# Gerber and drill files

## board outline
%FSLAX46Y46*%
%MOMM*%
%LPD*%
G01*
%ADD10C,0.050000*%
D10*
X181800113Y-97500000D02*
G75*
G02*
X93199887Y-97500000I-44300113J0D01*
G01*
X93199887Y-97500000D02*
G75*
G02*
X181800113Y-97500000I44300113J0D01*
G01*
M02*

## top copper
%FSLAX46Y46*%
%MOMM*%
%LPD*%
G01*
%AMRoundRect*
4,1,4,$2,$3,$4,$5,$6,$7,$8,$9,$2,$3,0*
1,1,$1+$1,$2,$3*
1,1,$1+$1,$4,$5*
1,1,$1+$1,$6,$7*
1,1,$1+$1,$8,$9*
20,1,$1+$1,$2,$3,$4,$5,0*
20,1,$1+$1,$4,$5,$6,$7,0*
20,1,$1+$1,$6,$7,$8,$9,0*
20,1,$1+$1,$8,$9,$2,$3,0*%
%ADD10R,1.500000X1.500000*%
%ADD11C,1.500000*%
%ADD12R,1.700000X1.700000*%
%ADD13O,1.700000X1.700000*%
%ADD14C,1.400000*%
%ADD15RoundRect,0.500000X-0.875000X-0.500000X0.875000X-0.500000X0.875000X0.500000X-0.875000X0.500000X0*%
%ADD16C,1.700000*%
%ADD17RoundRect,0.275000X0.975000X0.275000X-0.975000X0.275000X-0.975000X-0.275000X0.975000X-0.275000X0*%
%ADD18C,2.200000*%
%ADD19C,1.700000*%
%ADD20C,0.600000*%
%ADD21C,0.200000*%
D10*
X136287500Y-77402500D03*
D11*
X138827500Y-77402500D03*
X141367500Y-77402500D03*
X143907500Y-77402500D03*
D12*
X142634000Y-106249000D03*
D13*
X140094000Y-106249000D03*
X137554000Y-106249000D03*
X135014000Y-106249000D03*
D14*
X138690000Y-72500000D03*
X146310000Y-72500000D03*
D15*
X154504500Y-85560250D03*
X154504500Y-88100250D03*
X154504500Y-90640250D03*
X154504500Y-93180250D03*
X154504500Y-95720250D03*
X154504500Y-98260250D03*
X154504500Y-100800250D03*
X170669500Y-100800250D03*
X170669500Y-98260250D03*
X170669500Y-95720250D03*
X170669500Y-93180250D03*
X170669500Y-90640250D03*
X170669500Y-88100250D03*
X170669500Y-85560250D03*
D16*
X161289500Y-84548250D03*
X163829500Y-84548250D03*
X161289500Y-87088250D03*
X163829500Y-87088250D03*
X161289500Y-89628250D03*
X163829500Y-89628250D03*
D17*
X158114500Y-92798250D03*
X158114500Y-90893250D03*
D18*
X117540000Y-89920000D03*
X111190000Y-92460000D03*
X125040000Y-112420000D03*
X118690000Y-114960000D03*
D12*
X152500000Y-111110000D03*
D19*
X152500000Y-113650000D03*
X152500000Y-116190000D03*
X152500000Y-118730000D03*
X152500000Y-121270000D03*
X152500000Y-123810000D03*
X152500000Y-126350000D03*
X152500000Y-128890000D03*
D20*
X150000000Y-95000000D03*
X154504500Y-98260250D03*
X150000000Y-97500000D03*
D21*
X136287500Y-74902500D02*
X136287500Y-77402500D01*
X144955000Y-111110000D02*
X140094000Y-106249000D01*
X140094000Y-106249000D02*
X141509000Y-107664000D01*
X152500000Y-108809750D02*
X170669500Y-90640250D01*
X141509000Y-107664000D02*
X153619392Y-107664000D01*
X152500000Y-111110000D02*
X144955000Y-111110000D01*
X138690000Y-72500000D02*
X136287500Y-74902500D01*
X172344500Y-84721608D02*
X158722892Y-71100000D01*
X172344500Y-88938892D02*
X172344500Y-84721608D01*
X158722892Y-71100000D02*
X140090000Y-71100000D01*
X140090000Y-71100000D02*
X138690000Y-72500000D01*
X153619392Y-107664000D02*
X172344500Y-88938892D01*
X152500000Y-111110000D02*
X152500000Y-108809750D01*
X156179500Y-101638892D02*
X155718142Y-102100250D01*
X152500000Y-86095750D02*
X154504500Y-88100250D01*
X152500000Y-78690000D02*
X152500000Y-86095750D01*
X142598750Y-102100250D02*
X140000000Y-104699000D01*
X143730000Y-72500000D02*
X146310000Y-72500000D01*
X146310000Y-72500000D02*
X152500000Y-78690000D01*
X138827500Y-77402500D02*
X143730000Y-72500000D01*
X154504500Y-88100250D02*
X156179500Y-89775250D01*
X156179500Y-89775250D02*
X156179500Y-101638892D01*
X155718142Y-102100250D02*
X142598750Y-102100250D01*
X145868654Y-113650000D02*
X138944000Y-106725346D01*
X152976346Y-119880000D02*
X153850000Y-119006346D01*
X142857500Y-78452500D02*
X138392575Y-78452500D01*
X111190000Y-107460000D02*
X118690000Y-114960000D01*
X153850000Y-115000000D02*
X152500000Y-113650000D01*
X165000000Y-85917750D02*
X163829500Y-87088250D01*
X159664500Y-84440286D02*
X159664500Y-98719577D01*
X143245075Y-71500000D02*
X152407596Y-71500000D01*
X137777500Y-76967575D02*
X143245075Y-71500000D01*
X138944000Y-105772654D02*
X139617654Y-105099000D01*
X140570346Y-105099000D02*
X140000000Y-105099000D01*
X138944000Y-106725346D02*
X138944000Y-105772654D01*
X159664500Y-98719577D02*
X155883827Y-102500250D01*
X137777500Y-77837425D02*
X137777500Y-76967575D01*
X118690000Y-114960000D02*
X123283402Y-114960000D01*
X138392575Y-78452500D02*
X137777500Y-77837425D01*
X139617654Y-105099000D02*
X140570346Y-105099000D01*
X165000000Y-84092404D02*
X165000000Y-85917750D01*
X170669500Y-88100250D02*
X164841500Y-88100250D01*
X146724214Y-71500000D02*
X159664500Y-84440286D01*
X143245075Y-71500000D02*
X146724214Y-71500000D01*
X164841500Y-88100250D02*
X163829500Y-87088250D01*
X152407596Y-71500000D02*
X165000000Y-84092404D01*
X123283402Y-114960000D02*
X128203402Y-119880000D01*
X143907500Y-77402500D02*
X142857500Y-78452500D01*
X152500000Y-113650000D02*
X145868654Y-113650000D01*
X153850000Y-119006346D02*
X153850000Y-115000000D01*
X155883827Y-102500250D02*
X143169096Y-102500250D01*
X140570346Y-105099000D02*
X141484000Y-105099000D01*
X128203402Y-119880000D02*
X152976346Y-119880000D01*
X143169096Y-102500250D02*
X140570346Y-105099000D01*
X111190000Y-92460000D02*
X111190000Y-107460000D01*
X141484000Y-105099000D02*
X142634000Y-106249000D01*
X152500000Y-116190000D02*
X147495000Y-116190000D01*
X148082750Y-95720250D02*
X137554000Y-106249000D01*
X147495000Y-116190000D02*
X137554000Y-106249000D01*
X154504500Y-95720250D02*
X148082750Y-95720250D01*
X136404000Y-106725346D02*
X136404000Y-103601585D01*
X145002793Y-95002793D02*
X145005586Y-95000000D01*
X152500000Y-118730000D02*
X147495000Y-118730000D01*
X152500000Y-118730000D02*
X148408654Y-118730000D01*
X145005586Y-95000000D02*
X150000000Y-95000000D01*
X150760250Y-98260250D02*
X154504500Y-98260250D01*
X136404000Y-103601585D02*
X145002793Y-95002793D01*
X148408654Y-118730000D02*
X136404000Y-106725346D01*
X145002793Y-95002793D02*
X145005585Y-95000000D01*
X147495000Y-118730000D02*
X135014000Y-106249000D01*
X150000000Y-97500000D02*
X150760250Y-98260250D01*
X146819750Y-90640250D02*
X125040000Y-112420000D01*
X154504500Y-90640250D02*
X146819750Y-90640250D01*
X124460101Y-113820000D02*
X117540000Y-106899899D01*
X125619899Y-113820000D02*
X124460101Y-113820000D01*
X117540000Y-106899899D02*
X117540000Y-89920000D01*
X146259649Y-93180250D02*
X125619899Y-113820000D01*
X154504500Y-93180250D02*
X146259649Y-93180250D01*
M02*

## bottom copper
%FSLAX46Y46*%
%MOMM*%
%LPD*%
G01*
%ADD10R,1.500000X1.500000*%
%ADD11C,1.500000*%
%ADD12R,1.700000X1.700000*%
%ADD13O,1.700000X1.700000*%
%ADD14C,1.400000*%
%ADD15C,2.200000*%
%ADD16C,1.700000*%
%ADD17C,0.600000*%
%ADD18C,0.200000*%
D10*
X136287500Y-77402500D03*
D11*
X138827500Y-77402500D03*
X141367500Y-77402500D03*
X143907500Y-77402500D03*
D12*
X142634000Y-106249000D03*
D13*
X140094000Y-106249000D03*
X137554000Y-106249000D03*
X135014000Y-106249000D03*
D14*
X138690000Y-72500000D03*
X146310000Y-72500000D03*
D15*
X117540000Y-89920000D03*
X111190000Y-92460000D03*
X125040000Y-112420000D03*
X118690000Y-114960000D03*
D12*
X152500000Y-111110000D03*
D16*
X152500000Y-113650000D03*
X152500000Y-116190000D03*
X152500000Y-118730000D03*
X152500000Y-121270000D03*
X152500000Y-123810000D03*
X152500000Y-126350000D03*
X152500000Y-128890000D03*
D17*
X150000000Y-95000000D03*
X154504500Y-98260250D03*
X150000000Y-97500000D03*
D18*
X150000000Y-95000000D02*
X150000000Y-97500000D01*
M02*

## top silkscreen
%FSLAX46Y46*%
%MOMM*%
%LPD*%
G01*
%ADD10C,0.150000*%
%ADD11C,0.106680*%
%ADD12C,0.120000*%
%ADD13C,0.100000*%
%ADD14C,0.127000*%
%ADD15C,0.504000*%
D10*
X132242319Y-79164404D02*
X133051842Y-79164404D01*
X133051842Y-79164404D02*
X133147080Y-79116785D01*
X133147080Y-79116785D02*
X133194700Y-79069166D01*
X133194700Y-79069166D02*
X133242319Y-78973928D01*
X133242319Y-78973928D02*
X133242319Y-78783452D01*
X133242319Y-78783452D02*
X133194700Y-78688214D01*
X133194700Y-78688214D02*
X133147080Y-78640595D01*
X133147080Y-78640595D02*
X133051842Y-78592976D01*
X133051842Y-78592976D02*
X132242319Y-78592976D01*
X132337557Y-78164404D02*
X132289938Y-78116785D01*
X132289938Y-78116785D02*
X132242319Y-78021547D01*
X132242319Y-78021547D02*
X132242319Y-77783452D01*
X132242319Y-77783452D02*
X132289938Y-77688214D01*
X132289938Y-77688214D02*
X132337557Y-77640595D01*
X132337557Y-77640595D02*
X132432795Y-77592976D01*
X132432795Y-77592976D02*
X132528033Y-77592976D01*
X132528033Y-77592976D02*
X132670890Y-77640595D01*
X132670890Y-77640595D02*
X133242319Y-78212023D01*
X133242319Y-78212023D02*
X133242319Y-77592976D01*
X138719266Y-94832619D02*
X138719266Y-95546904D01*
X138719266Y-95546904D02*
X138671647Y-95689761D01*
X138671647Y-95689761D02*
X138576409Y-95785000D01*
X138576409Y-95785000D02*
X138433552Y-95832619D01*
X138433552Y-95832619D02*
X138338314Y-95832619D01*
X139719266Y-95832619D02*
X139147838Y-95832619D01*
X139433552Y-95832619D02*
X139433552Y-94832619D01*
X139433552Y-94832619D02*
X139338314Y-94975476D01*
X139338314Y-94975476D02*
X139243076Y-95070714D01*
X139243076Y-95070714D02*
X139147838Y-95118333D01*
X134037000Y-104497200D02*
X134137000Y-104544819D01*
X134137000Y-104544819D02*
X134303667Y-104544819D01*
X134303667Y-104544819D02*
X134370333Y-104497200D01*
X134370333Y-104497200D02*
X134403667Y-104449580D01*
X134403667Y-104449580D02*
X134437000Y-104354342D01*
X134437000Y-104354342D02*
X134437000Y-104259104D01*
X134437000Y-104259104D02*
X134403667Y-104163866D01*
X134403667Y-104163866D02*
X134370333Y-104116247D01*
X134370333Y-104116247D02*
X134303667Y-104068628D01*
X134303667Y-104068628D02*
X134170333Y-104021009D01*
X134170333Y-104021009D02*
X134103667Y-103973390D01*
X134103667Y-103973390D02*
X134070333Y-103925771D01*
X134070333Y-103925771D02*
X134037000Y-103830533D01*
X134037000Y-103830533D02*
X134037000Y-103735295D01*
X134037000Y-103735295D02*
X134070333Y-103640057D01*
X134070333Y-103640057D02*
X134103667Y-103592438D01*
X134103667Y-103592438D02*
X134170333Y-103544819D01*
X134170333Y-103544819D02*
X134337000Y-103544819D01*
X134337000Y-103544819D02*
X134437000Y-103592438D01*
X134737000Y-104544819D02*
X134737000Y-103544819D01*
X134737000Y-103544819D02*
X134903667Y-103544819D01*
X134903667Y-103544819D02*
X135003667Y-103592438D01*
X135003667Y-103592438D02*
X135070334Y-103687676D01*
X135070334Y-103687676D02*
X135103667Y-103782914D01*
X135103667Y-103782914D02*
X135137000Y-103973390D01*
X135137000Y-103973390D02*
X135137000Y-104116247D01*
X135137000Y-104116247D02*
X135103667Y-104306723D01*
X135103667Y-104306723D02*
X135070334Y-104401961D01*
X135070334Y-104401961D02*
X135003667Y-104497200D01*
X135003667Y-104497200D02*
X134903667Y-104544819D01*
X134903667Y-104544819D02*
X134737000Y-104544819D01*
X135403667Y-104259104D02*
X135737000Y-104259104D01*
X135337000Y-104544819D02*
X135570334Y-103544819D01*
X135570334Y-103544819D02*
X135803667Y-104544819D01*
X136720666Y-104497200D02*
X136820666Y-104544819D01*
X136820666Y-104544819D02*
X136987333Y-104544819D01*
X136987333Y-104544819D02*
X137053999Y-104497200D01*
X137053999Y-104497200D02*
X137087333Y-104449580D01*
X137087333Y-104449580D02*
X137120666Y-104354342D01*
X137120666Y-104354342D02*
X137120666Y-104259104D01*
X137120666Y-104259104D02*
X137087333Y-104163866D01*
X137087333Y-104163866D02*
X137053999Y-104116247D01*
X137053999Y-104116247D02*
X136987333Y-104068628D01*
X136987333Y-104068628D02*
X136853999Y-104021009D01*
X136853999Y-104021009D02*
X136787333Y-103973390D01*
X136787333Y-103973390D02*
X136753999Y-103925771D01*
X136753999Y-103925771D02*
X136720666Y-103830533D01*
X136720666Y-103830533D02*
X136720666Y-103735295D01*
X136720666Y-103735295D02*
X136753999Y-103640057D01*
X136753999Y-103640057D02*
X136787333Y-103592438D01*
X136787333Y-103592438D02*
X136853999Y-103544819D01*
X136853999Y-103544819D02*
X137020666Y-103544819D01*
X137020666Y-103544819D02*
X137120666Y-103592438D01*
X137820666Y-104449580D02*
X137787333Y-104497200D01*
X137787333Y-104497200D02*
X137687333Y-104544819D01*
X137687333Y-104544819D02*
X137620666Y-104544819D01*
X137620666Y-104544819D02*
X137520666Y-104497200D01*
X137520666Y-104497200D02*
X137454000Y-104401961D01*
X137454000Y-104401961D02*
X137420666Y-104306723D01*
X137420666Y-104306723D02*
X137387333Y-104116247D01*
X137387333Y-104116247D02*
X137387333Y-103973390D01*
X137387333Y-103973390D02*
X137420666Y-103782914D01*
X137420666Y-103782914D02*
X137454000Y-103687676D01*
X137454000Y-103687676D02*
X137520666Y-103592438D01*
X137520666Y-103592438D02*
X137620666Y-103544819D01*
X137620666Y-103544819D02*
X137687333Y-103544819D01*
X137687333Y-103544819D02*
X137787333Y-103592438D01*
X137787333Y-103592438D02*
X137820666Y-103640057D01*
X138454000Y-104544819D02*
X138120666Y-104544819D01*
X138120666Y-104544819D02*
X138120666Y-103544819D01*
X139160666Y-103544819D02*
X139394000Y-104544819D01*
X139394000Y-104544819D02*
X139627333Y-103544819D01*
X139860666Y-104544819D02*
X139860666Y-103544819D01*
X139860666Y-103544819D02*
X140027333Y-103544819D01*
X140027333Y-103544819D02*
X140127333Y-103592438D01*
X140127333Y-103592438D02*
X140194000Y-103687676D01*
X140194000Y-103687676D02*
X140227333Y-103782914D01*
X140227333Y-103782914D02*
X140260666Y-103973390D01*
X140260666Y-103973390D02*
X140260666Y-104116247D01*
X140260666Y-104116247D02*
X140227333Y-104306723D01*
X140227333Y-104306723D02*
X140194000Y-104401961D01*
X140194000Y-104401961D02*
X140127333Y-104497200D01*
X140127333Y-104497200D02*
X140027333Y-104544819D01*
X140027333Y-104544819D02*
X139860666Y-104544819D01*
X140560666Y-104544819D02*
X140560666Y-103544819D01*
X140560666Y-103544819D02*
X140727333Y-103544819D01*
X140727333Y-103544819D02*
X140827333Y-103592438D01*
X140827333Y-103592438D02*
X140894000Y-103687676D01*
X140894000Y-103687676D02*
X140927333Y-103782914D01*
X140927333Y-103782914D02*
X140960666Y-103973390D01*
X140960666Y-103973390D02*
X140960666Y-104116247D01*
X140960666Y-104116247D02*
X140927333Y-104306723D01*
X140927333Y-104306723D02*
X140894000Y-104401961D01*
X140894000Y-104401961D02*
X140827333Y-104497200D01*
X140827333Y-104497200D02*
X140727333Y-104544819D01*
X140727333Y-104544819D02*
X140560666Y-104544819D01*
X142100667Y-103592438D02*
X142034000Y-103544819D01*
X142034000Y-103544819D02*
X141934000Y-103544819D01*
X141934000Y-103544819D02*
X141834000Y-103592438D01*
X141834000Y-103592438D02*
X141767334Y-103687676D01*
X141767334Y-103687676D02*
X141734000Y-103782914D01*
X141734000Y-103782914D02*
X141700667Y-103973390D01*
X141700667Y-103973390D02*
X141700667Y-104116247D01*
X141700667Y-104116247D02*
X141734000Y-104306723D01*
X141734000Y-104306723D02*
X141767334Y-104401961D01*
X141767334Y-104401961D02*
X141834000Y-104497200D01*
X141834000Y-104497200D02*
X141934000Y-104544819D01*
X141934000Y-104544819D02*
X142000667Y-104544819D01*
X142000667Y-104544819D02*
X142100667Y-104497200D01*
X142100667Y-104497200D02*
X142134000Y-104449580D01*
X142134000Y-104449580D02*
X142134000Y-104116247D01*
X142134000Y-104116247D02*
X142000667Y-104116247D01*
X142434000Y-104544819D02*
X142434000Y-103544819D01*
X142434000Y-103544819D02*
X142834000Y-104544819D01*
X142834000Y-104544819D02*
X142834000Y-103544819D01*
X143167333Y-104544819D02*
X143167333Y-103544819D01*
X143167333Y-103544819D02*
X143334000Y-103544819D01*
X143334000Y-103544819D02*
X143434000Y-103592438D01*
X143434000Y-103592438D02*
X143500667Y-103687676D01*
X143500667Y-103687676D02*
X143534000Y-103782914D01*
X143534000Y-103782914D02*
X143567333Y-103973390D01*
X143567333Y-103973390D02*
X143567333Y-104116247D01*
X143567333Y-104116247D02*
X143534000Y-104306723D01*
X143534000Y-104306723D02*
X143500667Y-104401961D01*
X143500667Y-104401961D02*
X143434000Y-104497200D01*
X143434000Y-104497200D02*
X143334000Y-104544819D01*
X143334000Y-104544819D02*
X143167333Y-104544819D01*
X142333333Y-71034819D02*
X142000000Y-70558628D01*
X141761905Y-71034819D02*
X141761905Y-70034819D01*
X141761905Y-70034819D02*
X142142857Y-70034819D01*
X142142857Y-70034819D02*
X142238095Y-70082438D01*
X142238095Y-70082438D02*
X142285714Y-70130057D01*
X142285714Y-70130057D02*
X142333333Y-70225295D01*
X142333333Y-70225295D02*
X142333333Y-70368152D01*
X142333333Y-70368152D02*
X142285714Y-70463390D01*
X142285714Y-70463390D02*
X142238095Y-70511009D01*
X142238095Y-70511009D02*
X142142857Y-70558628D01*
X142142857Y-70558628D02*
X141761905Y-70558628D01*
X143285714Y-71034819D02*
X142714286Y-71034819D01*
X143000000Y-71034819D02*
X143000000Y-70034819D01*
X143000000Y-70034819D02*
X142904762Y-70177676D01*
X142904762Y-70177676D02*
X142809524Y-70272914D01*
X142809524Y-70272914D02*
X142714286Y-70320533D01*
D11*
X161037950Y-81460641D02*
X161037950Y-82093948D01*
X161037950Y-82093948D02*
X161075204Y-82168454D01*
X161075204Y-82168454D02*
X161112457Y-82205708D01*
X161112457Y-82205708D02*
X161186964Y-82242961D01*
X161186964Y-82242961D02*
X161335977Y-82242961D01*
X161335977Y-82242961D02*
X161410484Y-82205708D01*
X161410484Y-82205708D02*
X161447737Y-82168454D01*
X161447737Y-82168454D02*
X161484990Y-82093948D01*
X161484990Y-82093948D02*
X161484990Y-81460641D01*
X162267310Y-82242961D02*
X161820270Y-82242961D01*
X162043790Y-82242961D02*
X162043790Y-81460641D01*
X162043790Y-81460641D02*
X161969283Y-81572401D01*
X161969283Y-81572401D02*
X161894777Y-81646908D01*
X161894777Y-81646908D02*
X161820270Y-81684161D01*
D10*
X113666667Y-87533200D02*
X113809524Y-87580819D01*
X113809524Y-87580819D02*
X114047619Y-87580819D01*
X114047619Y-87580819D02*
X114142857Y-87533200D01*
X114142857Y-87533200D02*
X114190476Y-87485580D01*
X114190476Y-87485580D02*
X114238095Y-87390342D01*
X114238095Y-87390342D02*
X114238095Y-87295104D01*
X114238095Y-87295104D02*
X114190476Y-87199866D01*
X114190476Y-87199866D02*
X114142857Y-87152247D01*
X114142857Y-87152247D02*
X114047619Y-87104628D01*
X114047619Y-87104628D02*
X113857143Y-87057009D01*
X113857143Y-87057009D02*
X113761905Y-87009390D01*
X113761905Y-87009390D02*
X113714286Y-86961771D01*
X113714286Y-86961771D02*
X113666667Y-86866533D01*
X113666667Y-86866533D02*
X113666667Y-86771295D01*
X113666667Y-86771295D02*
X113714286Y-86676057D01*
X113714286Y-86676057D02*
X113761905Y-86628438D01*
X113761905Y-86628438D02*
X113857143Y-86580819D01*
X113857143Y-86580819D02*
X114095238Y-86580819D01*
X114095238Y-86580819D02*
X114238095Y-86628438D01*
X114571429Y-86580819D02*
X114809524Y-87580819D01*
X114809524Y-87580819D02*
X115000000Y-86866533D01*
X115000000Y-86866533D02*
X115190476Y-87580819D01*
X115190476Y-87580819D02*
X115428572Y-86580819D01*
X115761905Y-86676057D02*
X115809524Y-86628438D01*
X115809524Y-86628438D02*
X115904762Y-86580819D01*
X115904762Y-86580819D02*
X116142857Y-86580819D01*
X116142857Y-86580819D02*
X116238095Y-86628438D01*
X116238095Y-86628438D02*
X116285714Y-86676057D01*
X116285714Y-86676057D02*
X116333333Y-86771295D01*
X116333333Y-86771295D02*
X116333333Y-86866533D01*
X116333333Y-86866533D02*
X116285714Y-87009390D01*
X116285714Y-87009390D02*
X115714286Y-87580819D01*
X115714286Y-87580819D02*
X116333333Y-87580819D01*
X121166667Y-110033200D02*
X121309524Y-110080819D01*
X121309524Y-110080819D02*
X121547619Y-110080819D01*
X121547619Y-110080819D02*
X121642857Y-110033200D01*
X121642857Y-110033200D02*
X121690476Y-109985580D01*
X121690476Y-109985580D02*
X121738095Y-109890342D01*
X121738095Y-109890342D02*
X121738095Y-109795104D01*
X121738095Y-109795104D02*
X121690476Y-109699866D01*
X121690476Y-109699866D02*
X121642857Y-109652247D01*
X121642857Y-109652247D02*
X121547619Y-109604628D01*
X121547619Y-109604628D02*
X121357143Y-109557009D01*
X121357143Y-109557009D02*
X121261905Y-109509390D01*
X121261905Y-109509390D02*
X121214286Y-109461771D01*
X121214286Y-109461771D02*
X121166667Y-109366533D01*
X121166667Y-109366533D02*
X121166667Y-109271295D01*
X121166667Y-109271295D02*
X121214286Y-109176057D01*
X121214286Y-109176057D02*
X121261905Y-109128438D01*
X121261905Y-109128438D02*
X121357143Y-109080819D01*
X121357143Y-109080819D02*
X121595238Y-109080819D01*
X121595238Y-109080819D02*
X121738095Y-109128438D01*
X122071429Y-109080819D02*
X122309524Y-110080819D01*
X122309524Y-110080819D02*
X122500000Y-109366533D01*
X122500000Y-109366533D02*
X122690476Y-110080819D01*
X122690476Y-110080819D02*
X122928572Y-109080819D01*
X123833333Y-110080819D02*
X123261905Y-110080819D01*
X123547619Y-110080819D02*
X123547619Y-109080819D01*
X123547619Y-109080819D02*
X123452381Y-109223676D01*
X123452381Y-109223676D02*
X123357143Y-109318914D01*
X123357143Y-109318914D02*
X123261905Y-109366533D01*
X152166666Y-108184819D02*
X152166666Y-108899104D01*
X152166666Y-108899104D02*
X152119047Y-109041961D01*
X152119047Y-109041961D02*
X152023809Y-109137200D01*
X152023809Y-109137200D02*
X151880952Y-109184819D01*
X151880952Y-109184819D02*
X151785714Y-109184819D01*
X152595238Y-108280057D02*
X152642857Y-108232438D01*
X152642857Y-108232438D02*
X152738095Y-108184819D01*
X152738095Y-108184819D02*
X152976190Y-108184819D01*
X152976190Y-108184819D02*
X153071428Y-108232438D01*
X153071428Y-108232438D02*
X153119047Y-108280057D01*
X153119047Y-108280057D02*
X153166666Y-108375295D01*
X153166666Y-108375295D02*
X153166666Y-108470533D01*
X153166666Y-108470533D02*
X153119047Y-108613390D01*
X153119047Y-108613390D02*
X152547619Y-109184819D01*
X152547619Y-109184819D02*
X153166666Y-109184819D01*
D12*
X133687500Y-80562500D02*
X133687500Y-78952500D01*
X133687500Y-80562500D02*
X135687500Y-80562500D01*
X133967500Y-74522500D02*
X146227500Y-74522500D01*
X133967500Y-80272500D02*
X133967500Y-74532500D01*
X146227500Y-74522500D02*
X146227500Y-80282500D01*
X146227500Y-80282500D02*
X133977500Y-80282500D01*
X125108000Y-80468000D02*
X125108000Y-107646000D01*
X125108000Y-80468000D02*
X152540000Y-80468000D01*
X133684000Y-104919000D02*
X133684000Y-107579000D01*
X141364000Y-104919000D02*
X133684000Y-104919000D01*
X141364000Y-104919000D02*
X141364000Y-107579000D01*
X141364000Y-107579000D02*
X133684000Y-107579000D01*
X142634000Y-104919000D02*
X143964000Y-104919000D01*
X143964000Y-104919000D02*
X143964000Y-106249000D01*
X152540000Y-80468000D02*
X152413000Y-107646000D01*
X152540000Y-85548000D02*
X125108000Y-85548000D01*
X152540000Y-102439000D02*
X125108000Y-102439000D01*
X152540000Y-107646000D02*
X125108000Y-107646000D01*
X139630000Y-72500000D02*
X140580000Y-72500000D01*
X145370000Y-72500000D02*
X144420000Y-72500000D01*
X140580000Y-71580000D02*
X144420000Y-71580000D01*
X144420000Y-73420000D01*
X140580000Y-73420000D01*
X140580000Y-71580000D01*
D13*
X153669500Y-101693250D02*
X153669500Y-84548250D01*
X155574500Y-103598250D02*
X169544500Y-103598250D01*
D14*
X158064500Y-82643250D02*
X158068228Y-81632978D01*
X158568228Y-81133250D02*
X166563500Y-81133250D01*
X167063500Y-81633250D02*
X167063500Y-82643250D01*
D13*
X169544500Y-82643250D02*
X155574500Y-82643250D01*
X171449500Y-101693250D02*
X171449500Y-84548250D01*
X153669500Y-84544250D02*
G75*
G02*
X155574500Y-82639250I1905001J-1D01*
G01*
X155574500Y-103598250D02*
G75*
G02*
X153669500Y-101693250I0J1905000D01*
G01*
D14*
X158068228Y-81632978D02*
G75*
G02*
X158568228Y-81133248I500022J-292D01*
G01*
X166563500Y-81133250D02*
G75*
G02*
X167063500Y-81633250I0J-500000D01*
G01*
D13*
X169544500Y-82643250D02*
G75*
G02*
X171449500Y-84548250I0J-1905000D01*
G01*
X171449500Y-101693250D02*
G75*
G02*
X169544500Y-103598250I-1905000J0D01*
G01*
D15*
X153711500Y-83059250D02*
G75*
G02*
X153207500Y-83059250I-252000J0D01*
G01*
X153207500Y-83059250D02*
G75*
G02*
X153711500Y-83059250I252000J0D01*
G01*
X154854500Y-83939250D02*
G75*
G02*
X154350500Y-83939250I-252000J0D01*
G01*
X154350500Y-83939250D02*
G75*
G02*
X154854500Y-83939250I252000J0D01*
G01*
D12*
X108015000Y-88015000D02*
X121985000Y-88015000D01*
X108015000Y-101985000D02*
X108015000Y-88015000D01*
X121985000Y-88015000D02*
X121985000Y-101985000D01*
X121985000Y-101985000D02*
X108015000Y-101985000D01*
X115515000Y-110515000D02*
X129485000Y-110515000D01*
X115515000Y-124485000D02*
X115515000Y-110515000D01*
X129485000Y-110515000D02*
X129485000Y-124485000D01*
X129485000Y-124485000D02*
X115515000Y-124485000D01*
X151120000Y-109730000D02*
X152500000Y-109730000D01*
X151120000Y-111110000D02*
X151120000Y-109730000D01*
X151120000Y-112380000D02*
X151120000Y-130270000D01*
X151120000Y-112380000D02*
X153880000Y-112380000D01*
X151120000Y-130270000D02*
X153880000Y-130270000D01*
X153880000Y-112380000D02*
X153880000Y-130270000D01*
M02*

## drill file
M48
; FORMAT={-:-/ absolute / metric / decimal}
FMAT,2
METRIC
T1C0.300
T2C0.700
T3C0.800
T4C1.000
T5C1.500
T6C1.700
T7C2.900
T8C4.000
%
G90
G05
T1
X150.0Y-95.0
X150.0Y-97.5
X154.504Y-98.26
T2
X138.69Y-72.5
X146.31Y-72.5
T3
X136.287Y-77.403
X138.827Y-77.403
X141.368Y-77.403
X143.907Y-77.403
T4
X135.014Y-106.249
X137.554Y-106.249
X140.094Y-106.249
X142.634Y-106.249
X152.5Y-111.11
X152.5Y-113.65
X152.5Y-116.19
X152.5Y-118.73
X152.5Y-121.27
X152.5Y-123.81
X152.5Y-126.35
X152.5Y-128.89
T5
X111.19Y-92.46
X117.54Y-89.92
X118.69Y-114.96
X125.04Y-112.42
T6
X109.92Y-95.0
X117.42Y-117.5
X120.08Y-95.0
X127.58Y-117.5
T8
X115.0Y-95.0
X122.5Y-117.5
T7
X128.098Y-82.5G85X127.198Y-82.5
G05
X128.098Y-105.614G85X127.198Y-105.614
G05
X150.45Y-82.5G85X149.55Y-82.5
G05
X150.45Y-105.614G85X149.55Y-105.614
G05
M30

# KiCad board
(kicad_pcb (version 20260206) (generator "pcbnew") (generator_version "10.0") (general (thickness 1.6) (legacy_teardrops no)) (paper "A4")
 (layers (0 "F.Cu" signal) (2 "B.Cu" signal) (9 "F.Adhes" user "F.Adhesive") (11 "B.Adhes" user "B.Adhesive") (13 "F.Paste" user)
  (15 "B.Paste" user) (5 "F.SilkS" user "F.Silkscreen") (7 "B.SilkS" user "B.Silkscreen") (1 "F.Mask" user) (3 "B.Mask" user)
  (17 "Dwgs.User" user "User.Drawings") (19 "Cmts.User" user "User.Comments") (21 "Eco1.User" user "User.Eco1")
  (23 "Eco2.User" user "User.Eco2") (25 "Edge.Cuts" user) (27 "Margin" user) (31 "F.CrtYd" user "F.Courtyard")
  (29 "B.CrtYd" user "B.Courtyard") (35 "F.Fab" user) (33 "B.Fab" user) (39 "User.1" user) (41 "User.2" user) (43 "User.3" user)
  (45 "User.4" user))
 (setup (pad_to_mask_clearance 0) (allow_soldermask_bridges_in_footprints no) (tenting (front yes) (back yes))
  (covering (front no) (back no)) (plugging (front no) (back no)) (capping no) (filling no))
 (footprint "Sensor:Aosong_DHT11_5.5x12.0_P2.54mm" (layer "F.Cu") (at 136.2875 77.4025 90)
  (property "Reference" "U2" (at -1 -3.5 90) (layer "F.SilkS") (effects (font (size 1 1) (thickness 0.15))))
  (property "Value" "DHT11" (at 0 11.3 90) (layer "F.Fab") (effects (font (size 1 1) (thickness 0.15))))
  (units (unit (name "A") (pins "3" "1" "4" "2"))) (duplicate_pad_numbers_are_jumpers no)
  (fp_line (start -3.16 -2.6) (end -1.55 -2.6) (stroke (width 0.12) (type solid)) (layer "F.SilkS"))
  (fp_line (start -3.16 -2.6) (end -3.16 -0.6) (stroke (width 0.12) (type solid)) (layer "F.SilkS"))
  (fp_line (start 2.88 -2.32) (end 2.88 9.94) (stroke (width 0.12) (type solid)) (layer "F.SilkS"))
  (fp_line (start -2.87 -2.32) (end 2.87 -2.32) (stroke (width 0.12) (type solid)) (layer "F.SilkS"))
  (fp_line (start 2.88 9.94) (end -2.88 9.94) (stroke (width 0.12) (type solid)) (layer "F.SilkS"))
  (fp_line (start -2.88 9.94) (end -2.88 -2.31) (stroke (width 0.12) (type solid)) (layer "F.SilkS"))
  (pad "1" thru_hole rect (at 0 0 90) (size 1.5 1.5) (drill 0.8) (layers "*.Cu" "*.Mask") (remove_unused_layers no) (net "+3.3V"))
  (pad "2" thru_hole circle (at 0 2.54 90) (size 1.5 1.5) (drill 0.8) (layers "*.Cu" "*.Mask") (remove_unused_layers no) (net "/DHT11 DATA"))
  (pad "3" thru_hole circle (at 0 5.08 90) (size 1.5 1.5) (drill 0.8) (layers "*.Cu" "*.Mask") (remove_unused_layers no)
   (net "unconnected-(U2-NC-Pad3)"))
  (pad "4" thru_hole circle (at 0 7.62 90) (size 1.5 1.5) (drill 0.8) (layers "*.Cu" "*.Mask") (remove_unused_layers no) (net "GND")))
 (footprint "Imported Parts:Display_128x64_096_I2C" (layer "F.Cu") (at 138.824 106.249 180)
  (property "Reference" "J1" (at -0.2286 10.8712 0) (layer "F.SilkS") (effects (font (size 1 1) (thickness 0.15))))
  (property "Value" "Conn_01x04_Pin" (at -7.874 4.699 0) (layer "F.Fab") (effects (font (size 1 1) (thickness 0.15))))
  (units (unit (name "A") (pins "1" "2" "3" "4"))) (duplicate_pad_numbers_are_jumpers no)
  (fp_line (start 13.716 25.781) (end 13.716 -1.397) (stroke (width 0.12) (type solid)) (layer "F.SilkS"))
  (fp_line (start 13.716 25.781) (end -13.716 25.781) (stroke (width 0.12) (type solid)) (layer "F.SilkS"))
  (fp_line (start 5.14 1.33) (end 5.14 -1.33) (stroke (width 0.12) (type solid)) (layer "F.SilkS"))
  (fp_line (start -2.54 1.33) (end 5.14 1.33) (stroke (width 0.12) (type solid)) (layer "F.SilkS"))
  (fp_line (start -2.54 1.33) (end -2.54 -1.33) (stroke (width 0.12) (type solid)) (layer "F.SilkS"))
  (fp_line (start -2.54 -1.33) (end 5.14 -1.33) (stroke (width 0.12) (type solid)) (layer "F.SilkS"))
  (fp_line (start -3.81 1.33) (end -5.14 1.33) (stroke (width 0.12) (type solid)) (layer "F.SilkS"))
  (fp_line (start -5.14 1.33) (end -5.14 0) (stroke (width 0.12) (type solid)) (layer "F.SilkS"))
  (fp_line (start -13.716 25.781) (end -13.589 -1.397) (stroke (width 0.12) (type solid)) (layer "F.SilkS"))
  (fp_line (start -13.716 20.701) (end 13.716 20.701) (stroke (width 0.12) (type solid)) (layer "F.SilkS"))
  (fp_line (start -13.716 3.81) (end 13.716 3.81) (stroke (width 0.12) (type solid)) (layer "F.SilkS"))
  (fp_line (start -13.716 -1.397) (end 13.716 -1.397) (stroke (width 0.12) (type solid)) (layer "F.SilkS"))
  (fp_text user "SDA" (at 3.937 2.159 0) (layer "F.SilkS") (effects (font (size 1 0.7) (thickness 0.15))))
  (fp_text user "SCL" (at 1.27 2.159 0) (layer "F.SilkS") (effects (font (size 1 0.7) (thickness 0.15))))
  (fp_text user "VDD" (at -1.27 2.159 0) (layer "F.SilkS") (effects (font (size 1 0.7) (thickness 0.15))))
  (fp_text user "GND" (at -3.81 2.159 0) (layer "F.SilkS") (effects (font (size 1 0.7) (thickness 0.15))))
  (pad "" np_thru_hole oval (at -11.176 0.635 180) (size 3.8 2.9) (drill oval 3.8 2.9) (layers "*.Cu" "*.Mask"))
  (pad "" np_thru_hole oval (at -11.176 23.749 180) (size 3.8 2.9) (drill oval 3.8 2.9) (layers "*.Cu" "*.Mask"))
  (pad "" np_thru_hole oval (at 11.176 0.635 180) (size 3.8 2.9) (drill oval 3.8 2.9) (layers "*.Cu" "*.Mask"))
  (pad "" np_thru_hole oval (at 11.176 23.749 180) (size 3.8 2.9) (drill oval 3.8 2.9) (layers "*.Cu" "*.Mask"))
  (pad "1" thru_hole rect (at -3.81 0 270) (size 1.7 1.7) (drill 1) (layers "*.Cu" "*.Mask") (remove_unused_layers no) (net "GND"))
  (pad "2" thru_hole oval (at -1.27 0 270) (size 1.7 1.7) (drill 1) (layers "*.Cu" "*.Mask") (remove_unused_layers no) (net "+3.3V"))
  (pad "3" thru_hole oval (at 1.27 0 270) (size 1.7 1.7) (drill 1) (layers "*.Cu" "*.Mask") (remove_unused_layers no) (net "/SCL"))
  (pad "4" thru_hole oval (at 3.81 0 270) (size 1.7 1.7) (drill 1) (layers "*.Cu" "*.Mask") (remove_unused_layers no) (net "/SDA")))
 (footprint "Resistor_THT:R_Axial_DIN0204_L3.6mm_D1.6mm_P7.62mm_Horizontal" (layer "F.Cu") (at 138.69 72.5)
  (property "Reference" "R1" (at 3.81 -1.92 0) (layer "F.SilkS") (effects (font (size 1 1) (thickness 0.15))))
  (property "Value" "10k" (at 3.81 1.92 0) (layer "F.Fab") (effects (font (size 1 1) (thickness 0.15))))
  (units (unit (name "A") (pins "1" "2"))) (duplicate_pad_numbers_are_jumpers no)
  (fp_line (start 0.94 0) (end 1.89 0) (stroke (width 0.12) (type solid)) (layer "F.SilkS"))
  (fp_line (start 6.68 0) (end 5.73 0) (stroke (width 0.12) (type solid)) (layer "F.SilkS"))
  (fp_rect (start 1.89 -0.92) (end 5.73 0.92) (stroke (width 0.12) (type solid)) (fill no) (layer "F.SilkS"))
  (pad "1" thru_hole circle (at 0 0) (size 1.4 1.4) (drill 0.7) (layers "*.Cu" "*.Mask") (remove_unused_layers no) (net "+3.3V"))
  (pad "2" thru_hole circle (at 7.62 0) (size 1.4 1.4) (drill 0.7) (layers "*.Cu" "*.Mask") (remove_unused_layers no) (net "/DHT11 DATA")))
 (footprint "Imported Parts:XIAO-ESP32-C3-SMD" (layer "F.Cu") (at 153.6695 103.68025)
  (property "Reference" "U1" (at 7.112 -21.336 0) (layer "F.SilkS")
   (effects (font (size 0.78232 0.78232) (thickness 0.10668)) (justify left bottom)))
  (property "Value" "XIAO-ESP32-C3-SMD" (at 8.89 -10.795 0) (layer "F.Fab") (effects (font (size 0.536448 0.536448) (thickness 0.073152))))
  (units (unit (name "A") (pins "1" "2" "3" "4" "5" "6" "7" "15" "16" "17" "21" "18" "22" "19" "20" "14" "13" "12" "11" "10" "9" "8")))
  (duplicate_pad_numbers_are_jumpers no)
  (fp_line (start 0 -1.987) (end 0 -19.132) (stroke (width 0.1) (type solid)) (layer "F.SilkS"))
  (fp_line (start 1.905 -0.082) (end 15.875 -0.082) (stroke (width 0.1) (type solid)) (layer "F.SilkS"))
  (fp_line (start 4.395 -21.037) (end 4.398728 -22.047272) (stroke (width 0.127) (type solid)) (layer "F.SilkS"))
  (fp_line (start 4.898728 -22.547) (end 12.894 -22.547) (stroke (width 0.127) (type solid)) (layer "F.SilkS"))
  (fp_line (start 13.394 -22.047) (end 13.394 -21.037) (stroke (width 0.127) (type solid)) (layer "F.SilkS"))
  (fp_line (start 15.875 -21.037) (end 1.905 -21.037) (stroke (width 0.1) (type solid)) (layer "F.SilkS"))
  (fp_line (start 17.78 -1.987) (end 17.78 -19.132) (stroke (width 0.1) (type solid)) (layer "F.SilkS"))
  (fp_arc (start 0 -19.136) (mid 0.557962 -20.483038) (end 1.905 -21.041) (stroke (width 0.1) (type solid)) (layer "F.SilkS"))
  (fp_arc (start 1.905 -0.082) (mid 0.557962 -0.639962) (end 0 -1.987) (stroke (width 0.1) (type solid)) (layer "F.SilkS"))
  (fp_arc (start 4.398728 -22.047272) (mid 4.545272 -22.40064) (end 4.898728 -22.547) (stroke (width 0.127) (type default))
   (layer "F.SilkS"))
  (fp_arc (start 12.894 -22.547) (mid 13.247553 -22.400553) (end 13.394 -22.047) (stroke (width 0.127) (type default)) (layer "F.SilkS"))
  (fp_arc (start 15.875 -21.037) (mid 17.222038 -20.479038) (end 17.78 -19.132) (stroke (width 0.1) (type solid)) (layer "F.SilkS"))
  (fp_arc (start 17.78 -1.987) (mid 17.222038 -0.639962) (end 15.875 -0.082) (stroke (width 0.1) (type solid)) (layer "F.SilkS"))
  (fp_circle (center -0.21 -20.621) (end -0.21 -20.875) (stroke (width 0.5) (type solid)) (fill yes) (layer "F.SilkS"))
  (fp_circle (center 0.933 -19.741) (end 0.933 -19.995) (stroke (width 0.5) (type solid)) (fill yes) (layer "F.SilkS"))
  (pad "1" smd roundrect (at 0.835 -18.12) (size 2.75 2) (layers "F.Cu" "F.Mask" "F.Paste") (roundrect_rratio 0.25)
   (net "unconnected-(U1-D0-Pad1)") (solder_mask_margin 0.0508) (thermal_bridge_angle 45))
  (pad "2" smd roundrect (at 0.835 -15.58) (size 2.75 2) (layers "F.Cu" "F.Mask" "F.Paste") (roundrect_rratio 0.25) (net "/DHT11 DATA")
   (solder_mask_margin 0.0508) (thermal_bridge_angle 45))
  (pad "3" smd roundrect (at 0.835 -13.04) (size 2.75 2) (layers "F.Cu" "F.Mask" "F.Paste") (roundrect_rratio 0.25) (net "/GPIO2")
   (solder_mask_margin 0.0508) (thermal_bridge_angle 45))
  (pad "4" smd roundrect (at 0.835 -10.5) (size 2.75 2) (layers "F.Cu" "F.Mask" "F.Paste") (roundrect_rratio 0.25) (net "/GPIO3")
   (solder_mask_margin 0.0508) (thermal_bridge_angle 45))
  (pad "5" smd roundrect (at 0.835 -7.96) (size 2.75 2) (layers "F.Cu" "F.Mask" "F.Paste") (roundrect_rratio 0.25) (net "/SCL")
   (solder_mask_margin 0.0508) (thermal_bridge_angle 45))
  (pad "6" smd roundrect (at 0.835 -5.42) (size 2.75 2) (layers "F.Cu" "F.Mask" "F.Paste") (roundrect_rratio 0.25) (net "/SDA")
   (solder_mask_margin 0.0508) (thermal_bridge_angle 45))
  (pad "7" smd roundrect (at 0.835 -2.88) (size 2.75 2) (layers "F.Cu" "F.Mask" "F.Paste") (roundrect_rratio 0.25)
   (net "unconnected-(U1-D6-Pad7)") (solder_mask_margin 0.0508) (thermal_bridge_angle 45))
  (pad "8" smd roundrect (at 17 -2.88) (size 2.75 2) (layers "F.Cu" "F.Mask" "F.Paste") (roundrect_rratio 0.25)
   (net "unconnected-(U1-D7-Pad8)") (solder_mask_margin 0.0508) (thermal_bridge_angle 45))
  (pad "9" smd roundrect (at 17 -5.42) (size 2.75 2) (layers "F.Cu" "F.Mask" "F.Paste") (roundrect_rratio 0.25)
   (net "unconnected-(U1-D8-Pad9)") (solder_mask_margin 0.0508) (thermal_bridge_angle 45))
  (pad "10" smd roundrect (at 17 -7.96) (size 2.75 2) (layers "F.Cu" "F.Mask" "F.Paste") (roundrect_rratio 0.25)
   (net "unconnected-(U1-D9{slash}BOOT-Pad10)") (solder_mask_margin 0.0508) (thermal_bridge_angle 45))
  (pad "11" smd roundrect (at 17 -10.5) (size 2.75 2) (layers "F.Cu" "F.Mask" "F.Paste") (roundrect_rratio 0.25)
   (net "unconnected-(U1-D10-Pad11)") (solder_mask_margin 0.0508) (thermal_bridge_angle 45))
  (pad "12" smd roundrect (at 17 -13.04) (size 2.75 2) (layers "F.Cu" "F.Mask" "F.Paste") (roundrect_rratio 0.25) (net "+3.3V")
   (solder_mask_margin 0.0508) (thermal_bridge_angle 45))
  (pad "13" smd roundrect (at 17 -15.58) (size 2.75 2) (layers "F.Cu" "F.Mask" "F.Paste") (roundrect_rratio 0.25) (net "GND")
   (solder_mask_margin 0.0508) (thermal_bridge_angle 45))
  (pad "14" smd roundrect (at 17 -18.12) (size 2.75 2) (layers "F.Cu" "F.Mask" "F.Paste") (roundrect_rratio 0.25) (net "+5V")
   (solder_mask_margin 0.0508) (thermal_bridge_angle 45))
  (pad "15" smd circle (at 7.62 -19.132) (size 1.7 1.7) (layers "F.Cu" "F.Mask" "F.Paste") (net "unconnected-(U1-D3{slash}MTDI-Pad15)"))
  (pad "16" smd circle (at 10.16 -19.132) (size 1.7 1.7) (layers "F.Cu" "F.Mask" "F.Paste") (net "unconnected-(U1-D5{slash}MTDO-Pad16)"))
  (pad "17" smd circle (at 7.62 -16.592) (size 1.7 1.7) (layers "F.Cu" "F.Mask" "F.Paste") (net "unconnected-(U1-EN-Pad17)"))
  (pad "18" smd circle (at 10.16 -16.592) (size 1.7 1.7) (layers "F.Cu" "F.Mask" "F.Paste") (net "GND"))
  (pad "19" smd circle (at 7.62 -14.052) (size 1.7 1.7) (layers "F.Cu" "F.Mask" "F.Paste") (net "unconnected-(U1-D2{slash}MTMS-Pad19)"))
  (pad "20" smd circle (at 10.16 -14.052) (size 1.7 1.7) (layers "F.Cu" "F.Mask" "F.Paste") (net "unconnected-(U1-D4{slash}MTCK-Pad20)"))
  (pad "21" smd roundrect (at 4.445 -10.882 180) (size 2.5 1.1) (layers "F.Cu" "F.Mask" "F.Paste") (roundrect_rratio 0.25)
   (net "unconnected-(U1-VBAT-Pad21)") (thermal_bridge_angle 45))
  (pad "22" smd roundrect (at 4.445 -12.787 180) (size 2.5 1.1) (layers "F.Cu" "F.Mask" "F.Paste") (roundrect_rratio 0.25)
   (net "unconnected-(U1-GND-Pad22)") (thermal_bridge_angle 45)))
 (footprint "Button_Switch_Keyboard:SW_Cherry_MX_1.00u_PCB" (layer "F.Cu") (at 117.54 89.92)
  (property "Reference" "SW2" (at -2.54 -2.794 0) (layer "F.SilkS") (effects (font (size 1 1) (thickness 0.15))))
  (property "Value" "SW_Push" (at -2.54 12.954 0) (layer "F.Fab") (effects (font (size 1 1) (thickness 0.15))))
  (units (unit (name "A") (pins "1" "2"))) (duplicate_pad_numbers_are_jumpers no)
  (fp_line (start -9.525 -1.905) (end 4.445 -1.905) (stroke (width 0.12) (type solid)) (layer "F.SilkS"))
  (fp_line (start -9.525 12.065) (end -9.525 -1.905) (stroke (width 0.12) (type solid)) (layer "F.SilkS"))
  (fp_line (start 4.445 -1.905) (end 4.445 12.065) (stroke (width 0.12) (type solid)) (layer "F.SilkS"))
  (fp_line (start 4.445 12.065) (end -9.525 12.065) (stroke (width 0.12) (type solid)) (layer "F.SilkS"))
  (pad "" np_thru_hole circle (at -7.62 5.08) (size 1.7 1.7) (drill 1.7) (layers "*.Cu" "*.Mask"))
  (pad "" np_thru_hole circle (at -2.54 5.08) (size 4 4) (drill 4) (layers "*.Cu" "*.Mask"))
  (pad "" np_thru_hole circle (at 2.54 5.08) (size 1.7 1.7) (drill 1.7) (layers "*.Cu" "*.Mask"))
  (pad "1" thru_hole circle (at 0 0) (size 2.2 2.2) (drill 1.5) (layers "*.Cu" "*.Mask") (remove_unused_layers no) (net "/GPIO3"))
  (pad "2" thru_hole circle (at -6.35 2.54) (size 2.2 2.2) (drill 1.5) (layers "*.Cu" "*.Mask") (remove_unused_layers no) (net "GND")))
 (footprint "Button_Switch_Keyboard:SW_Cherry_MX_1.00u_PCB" (layer "F.Cu") (at 125.04 112.42)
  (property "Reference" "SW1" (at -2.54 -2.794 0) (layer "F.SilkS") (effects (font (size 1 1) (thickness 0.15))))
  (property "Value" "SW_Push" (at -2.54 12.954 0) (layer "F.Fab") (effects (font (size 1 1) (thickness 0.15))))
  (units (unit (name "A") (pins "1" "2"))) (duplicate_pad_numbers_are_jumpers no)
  (fp_line (start -9.525 -1.905) (end 4.445 -1.905) (stroke (width 0.12) (type solid)) (layer "F.SilkS"))
  (fp_line (start -9.525 12.065) (end -9.525 -1.905) (stroke (width 0.12) (type solid)) (layer "F.SilkS"))
  (fp_line (start 4.445 -1.905) (end 4.445 12.065) (stroke (width 0.12) (type solid)) (layer "F.SilkS"))
  (fp_line (start 4.445 12.065) (end -9.525 12.065) (stroke (width 0.12) (type solid)) (layer "F.SilkS"))
  (pad "" np_thru_hole circle (at -7.62 5.08) (size 1.7 1.7) (drill 1.7) (layers "*.Cu" "*.Mask"))
  (pad "" np_thru_hole circle (at -2.54 5.08) (size 4 4) (drill 4) (layers "*.Cu" "*.Mask"))
  (pad "" np_thru_hole circle (at 2.54 5.08) (size 1.7 1.7) (drill 1.7) (layers "*.Cu" "*.Mask"))
  (pad "1" thru_hole circle (at 0 0) (size 2.2 2.2) (drill 1.5) (layers "*.Cu" "*.Mask") (remove_unused_layers no) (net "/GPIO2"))
  (pad "2" thru_hole circle (at -6.35 2.54) (size 2.2 2.2) (drill 1.5) (layers "*.Cu" "*.Mask") (remove_unused_layers no) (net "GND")))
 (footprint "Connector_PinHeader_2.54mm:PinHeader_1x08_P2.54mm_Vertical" (layer "F.Cu") (at 152.5 111.11)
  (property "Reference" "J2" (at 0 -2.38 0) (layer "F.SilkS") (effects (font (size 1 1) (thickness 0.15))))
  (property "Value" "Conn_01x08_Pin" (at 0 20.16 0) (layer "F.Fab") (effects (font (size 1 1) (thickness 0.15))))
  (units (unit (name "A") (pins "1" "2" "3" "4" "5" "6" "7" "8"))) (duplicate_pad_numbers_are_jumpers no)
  (fp_line (start -1.38 -1.38) (end 0 -1.38) (stroke (width 0.12) (type solid)) (layer "F.SilkS"))
  (fp_line (start -1.38 0) (end -1.38 -1.38) (stroke (width 0.12) (type solid)) (layer "F.SilkS"))
  (fp_line (start -1.38 1.27) (end -1.38 19.16) (stroke (width 0.12) (type solid)) (layer "F.SilkS"))
  (fp_line (start -1.38 1.27) (end 1.38 1.27) (stroke (width 0.12) (type solid)) (layer "F.SilkS"))
  (fp_line (start -1.38 19.16) (end 1.38 19.16) (stroke (width 0.12) (type solid)) (layer "F.SilkS"))
  (fp_line (start 1.38 1.27) (end 1.38 19.16) (stroke (width 0.12) (type solid)) (layer "F.SilkS"))
  (pad "1" thru_hole rect (at 0 0) (size 1.7 1.7) (drill 1) (layers "*.Cu" "*.Mask") (remove_unused_layers no) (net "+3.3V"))
  (pad "2" thru_hole circle (at 0 2.54) (size 1.7 1.7) (drill 1) (layers "*.Cu" "*.Mask") (remove_unused_layers no) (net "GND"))
  (pad "3" thru_hole circle (at 0 5.08) (size 1.7 1.7) (drill 1) (layers "*.Cu" "*.Mask") (remove_unused_layers no) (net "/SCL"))
  (pad "4" thru_hole circle (at 0 7.62) (size 1.7 1.7) (drill 1) (layers "*.Cu" "*.Mask") (remove_unused_layers no) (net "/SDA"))
  (pad "5" thru_hole circle (at 0 10.16) (size 1.7 1.7) (drill 1) (layers "*.Cu" "*.Mask") (remove_unused_layers no)
   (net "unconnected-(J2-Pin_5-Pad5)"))
  (pad "6" thru_hole circle (at 0 12.7) (size 1.7 1.7) (drill 1) (layers "*.Cu" "*.Mask") (remove_unused_layers no)
   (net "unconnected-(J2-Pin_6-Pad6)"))
  (pad "7" thru_hole circle (at 0 15.24) (size 1.7 1.7) (drill 1) (layers "*.Cu" "*.Mask") (remove_unused_layers no)
   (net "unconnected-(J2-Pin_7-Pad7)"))
  (pad "8" thru_hole circle (at 0 17.78) (size 1.7 1.7) (drill 1) (layers "*.Cu" "*.Mask") (remove_unused_layers no)
   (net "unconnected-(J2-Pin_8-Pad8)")))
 (gr_circle (center 137.5 97.5) (end 150 55) (stroke (width 0.05) (type default)) (fill no) (layer "Edge.Cuts"))
 (segment (start 136.2875 74.9025) (end 136.2875 77.4025) (width 0.2) (layer "F.Cu") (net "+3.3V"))
 (segment (start 144.955 111.11) (end 140.094 106.249) (width 0.2) (layer "F.Cu") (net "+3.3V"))
 (segment (start 140.094 106.249) (end 141.509 107.664) (width 0.2) (layer "F.Cu") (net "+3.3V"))
 (segment (start 152.5 108.80975) (end 170.6695 90.64025) (width 0.2) (layer "F.Cu") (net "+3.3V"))
 (segment (start 141.509 107.664) (end 153.619392 107.664) (width 0.2) (layer "F.Cu") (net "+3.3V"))
 (segment (start 152.5 111.11) (end 144.955 111.11) (width 0.2) (layer "F.Cu") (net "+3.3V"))
 (segment (start 138.69 72.5) (end 136.2875 74.9025) (width 0.2) (layer "F.Cu") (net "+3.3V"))
 (segment (start 172.3445 84.721608) (end 158.722892 71.1) (width 0.2) (layer "F.Cu") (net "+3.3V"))
 (segment (start 172.3445 88.938892) (end 172.3445 84.721608) (width 0.2) (layer "F.Cu") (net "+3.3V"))
 (segment (start 158.722892 71.1) (end 140.09 71.1) (width 0.2) (layer "F.Cu") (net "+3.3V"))
 (segment (start 140.09 71.1) (end 138.69 72.5) (width 0.2) (layer "F.Cu") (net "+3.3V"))
 (segment (start 153.619392 107.664) (end 172.3445 88.938892) (width 0.2) (layer "F.Cu") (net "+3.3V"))
 (segment (start 152.5 111.11) (end 152.5 108.80975) (width 0.2) (layer "F.Cu") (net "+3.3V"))
 (segment (start 156.1795 101.638892) (end 155.718142 102.10025) (width 0.2) (layer "F.Cu") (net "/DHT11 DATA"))
 (segment (start 152.5 86.09575) (end 154.5045 88.10025) (width 0.2) (layer "F.Cu") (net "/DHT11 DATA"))
 (segment (start 152.5 78.69) (end 152.5 86.09575) (width 0.2) (layer "F.Cu") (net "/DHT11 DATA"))
 (segment (start 142.59875 102.10025) (end 140 104.699) (width 0.2) (layer "F.Cu") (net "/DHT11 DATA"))
 (segment (start 143.73 72.5) (end 146.31 72.5) (width 0.2) (layer "F.Cu") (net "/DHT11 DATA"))
 (segment (start 146.31 72.5) (end 152.5 78.69) (width 0.2) (layer "F.Cu") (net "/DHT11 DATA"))
 (segment (start 138.8275 77.4025) (end 143.73 72.5) (width 0.2) (layer "F.Cu") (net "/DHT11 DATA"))
 (segment (start 154.5045 88.10025) (end 156.1795 89.77525) (width 0.2) (layer "F.Cu") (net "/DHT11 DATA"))
 (segment (start 156.1795 89.77525) (end 156.1795 101.638892) (width 0.2) (layer "F.Cu") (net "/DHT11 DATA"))
 (segment (start 155.718142 102.10025) (end 142.59875 102.10025) (width 0.2) (layer "F.Cu") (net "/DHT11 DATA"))
 (segment (start 145.868654 113.65) (end 138.944 106.725346) (width 0.2) (layer "F.Cu") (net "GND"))
 (segment (start 152.976346 119.88) (end 153.85 119.006346) (width 0.2) (layer "F.Cu") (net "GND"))
 (segment (start 142.8575 78.4525) (end 138.392575 78.4525) (width 0.2) (layer "F.Cu") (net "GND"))
 (segment (start 111.19 107.46) (end 118.69 114.96) (width 0.2) (layer "F.Cu") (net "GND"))
 (segment (start 153.85 115) (end 152.5 113.65) (width 0.2) (layer "F.Cu") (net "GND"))
 (segment (start 165 85.91775) (end 163.8295 87.08825) (width 0.2) (layer "F.Cu") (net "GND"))
 (segment (start 159.6645 84.440286) (end 159.6645 98.719577) (width 0.2) (layer "F.Cu") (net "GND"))
 (segment (start 143.245075 71.5) (end 152.407596 71.5) (width 0.2) (layer "F.Cu") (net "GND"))
 (segment (start 137.7775 76.967575) (end 143.245075 71.5) (width 0.2) (layer "F.Cu") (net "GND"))
 (segment (start 138.944 105.772654) (end 139.617654 105.099) (width 0.2) (layer "F.Cu") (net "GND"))
 (segment (start 140.570346 105.099) (end 140 105.099) (width 0.2) (layer "F.Cu") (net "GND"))
 (segment (start 138.944 106.725346) (end 138.944 105.772654) (width 0.2) (layer "F.Cu") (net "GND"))
 (segment (start 159.6645 98.719577) (end 155.883827 102.50025) (width 0.2) (layer "F.Cu") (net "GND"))
 (segment (start 137.7775 77.837425) (end 137.7775 76.967575) (width 0.2) (layer "F.Cu") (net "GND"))
 (segment (start 118.69 114.96) (end 123.283402 114.96) (width 0.2) (layer "F.Cu") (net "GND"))
 (segment (start 138.392575 78.4525) (end 137.7775 77.837425) (width 0.2) (layer "F.Cu") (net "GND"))
 (segment (start 139.617654 105.099) (end 140.570346 105.099) (width 0.2) (layer "F.Cu") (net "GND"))
 (segment (start 165 84.092404) (end 165 85.91775) (width 0.2) (layer "F.Cu") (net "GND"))
 (segment (start 170.6695 88.10025) (end 164.8415 88.10025) (width 0.2) (layer "F.Cu") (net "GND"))
 (segment (start 146.724214 71.5) (end 159.6645 84.440286) (width 0.2) (layer "F.Cu") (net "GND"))
 (segment (start 143.245075 71.5) (end 146.724214 71.5) (width 0.2) (layer "F.Cu") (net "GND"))
 (segment (start 164.8415 88.10025) (end 163.8295 87.08825) (width 0.2) (layer "F.Cu") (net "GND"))
 (segment (start 152.407596 71.5) (end 165 84.092404) (width 0.2) (layer "F.Cu") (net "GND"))
 (segment (start 123.283402 114.96) (end 128.203402 119.88) (width 0.2) (layer "F.Cu") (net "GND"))
 (segment (start 143.9075 77.4025) (end 142.8575 78.4525) (width 0.2) (layer "F.Cu") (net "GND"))
 (segment (start 152.5 113.65) (end 145.868654 113.65) (width 0.2) (layer "F.Cu") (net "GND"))
 (segment (start 153.85 119.006346) (end 153.85 115) (width 0.2) (layer "F.Cu") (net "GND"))
 (segment (start 155.883827 102.50025) (end 143.169096 102.50025) (width 0.2) (layer "F.Cu") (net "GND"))
 (segment (start 140.570346 105.099) (end 141.484 105.099) (width 0.2) (layer "F.Cu") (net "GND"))
 (segment (start 128.203402 119.88) (end 152.976346 119.88) (width 0.2) (layer "F.Cu") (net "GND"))
 (segment (start 143.169096 102.50025) (end 140.570346 105.099) (width 0.2) (layer "F.Cu") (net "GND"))
 (segment (start 111.19 92.46) (end 111.19 107.46) (width 0.2) (layer "F.Cu") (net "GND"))
 (segment (start 141.484 105.099) (end 142.634 106.249) (width 0.2) (layer "F.Cu") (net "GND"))
 (segment (start 152.5 116.19) (end 147.495 116.19) (width 0.2) (layer "F.Cu") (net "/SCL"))
 (segment (start 148.08275 95.72025) (end 137.554 106.249) (width 0.2) (layer "F.Cu") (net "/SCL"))
 (segment (start 147.495 116.19) (end 137.554 106.249) (width 0.2) (layer "F.Cu") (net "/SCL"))
 (segment (start 154.5045 95.72025) (end 148.08275 95.72025) (width 0.2) (layer "F.Cu") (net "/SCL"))
 (segment (start 136.404 106.725346) (end 136.404 103.601585) (width 0.2) (layer "F.Cu") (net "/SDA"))
 (segment (start 145.002793 95.002793) (end 145.005586 95) (width 0.2) (layer "F.Cu") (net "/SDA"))
 (segment (start 152.5 118.73) (end 147.495 118.73) (width 0.2) (layer "F.Cu") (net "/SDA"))
 (segment (start 152.5 118.73) (end 148.408654 118.73) (width 0.2) (layer "F.Cu") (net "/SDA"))
 (segment (start 145.005586 95) (end 150 95) (width 0.2) (layer "F.Cu") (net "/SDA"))
 (segment (start 150.76025 98.26025) (end 154.5045 98.26025) (width 0.2) (layer "F.Cu") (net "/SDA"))
 (segment (start 136.404 103.601585) (end 145.002793 95.002793) (width 0.2) (layer "F.Cu") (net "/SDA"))
 (segment (start 148.408654 118.73) (end 136.404 106.725346) (width 0.2) (layer "F.Cu") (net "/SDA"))
 (segment (start 145.002793 95.002793) (end 145.005585 95) (width 0.2) (layer "F.Cu") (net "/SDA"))
 (segment (start 147.495 118.73) (end 135.014 106.249) (width 0.2) (layer "F.Cu") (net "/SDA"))
 (segment (start 150 97.5) (end 150.76025 98.26025) (width 0.2) (layer "F.Cu") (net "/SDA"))
 (via (at 150 95) (size 0.6) (drill 0.3) (layers "F.Cu" "B.Cu") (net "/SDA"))
 (via (at 154.5045 98.26025) (size 0.6) (drill 0.3) (layers "F.Cu" "B.Cu") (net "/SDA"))
 (via (at 150 97.5) (size 0.6) (drill 0.3) (layers "F.Cu" "B.Cu") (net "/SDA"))
 (segment (start 150 95) (end 150 97.5) (width 0.2) (layer "B.Cu") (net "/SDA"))
 (segment (start 146.81975 90.64025) (end 125.04 112.42) (width 0.2) (layer "F.Cu") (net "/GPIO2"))
 (segment (start 154.5045 90.64025) (end 146.81975 90.64025) (width 0.2) (layer "F.Cu") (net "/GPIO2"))
 (segment (start 124.460101 113.82) (end 117.54 106.899899) (width 0.2) (layer "F.Cu") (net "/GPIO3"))
 (segment (start 125.619899 113.82) (end 124.460101 113.82) (width 0.2) (layer "F.Cu") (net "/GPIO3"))
 (segment (start 117.54 106.899899) (end 117.54 89.92) (width 0.2) (layer "F.Cu") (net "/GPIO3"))
 (segment (start 146.259649 93.18025) (end 125.619899 113.82) (width 0.2) (layer "F.Cu") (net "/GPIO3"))
 (segment (start 154.5045 93.18025) (end 146.259649 93.18025) (width 0.2) (layer "F.Cu") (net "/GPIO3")))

